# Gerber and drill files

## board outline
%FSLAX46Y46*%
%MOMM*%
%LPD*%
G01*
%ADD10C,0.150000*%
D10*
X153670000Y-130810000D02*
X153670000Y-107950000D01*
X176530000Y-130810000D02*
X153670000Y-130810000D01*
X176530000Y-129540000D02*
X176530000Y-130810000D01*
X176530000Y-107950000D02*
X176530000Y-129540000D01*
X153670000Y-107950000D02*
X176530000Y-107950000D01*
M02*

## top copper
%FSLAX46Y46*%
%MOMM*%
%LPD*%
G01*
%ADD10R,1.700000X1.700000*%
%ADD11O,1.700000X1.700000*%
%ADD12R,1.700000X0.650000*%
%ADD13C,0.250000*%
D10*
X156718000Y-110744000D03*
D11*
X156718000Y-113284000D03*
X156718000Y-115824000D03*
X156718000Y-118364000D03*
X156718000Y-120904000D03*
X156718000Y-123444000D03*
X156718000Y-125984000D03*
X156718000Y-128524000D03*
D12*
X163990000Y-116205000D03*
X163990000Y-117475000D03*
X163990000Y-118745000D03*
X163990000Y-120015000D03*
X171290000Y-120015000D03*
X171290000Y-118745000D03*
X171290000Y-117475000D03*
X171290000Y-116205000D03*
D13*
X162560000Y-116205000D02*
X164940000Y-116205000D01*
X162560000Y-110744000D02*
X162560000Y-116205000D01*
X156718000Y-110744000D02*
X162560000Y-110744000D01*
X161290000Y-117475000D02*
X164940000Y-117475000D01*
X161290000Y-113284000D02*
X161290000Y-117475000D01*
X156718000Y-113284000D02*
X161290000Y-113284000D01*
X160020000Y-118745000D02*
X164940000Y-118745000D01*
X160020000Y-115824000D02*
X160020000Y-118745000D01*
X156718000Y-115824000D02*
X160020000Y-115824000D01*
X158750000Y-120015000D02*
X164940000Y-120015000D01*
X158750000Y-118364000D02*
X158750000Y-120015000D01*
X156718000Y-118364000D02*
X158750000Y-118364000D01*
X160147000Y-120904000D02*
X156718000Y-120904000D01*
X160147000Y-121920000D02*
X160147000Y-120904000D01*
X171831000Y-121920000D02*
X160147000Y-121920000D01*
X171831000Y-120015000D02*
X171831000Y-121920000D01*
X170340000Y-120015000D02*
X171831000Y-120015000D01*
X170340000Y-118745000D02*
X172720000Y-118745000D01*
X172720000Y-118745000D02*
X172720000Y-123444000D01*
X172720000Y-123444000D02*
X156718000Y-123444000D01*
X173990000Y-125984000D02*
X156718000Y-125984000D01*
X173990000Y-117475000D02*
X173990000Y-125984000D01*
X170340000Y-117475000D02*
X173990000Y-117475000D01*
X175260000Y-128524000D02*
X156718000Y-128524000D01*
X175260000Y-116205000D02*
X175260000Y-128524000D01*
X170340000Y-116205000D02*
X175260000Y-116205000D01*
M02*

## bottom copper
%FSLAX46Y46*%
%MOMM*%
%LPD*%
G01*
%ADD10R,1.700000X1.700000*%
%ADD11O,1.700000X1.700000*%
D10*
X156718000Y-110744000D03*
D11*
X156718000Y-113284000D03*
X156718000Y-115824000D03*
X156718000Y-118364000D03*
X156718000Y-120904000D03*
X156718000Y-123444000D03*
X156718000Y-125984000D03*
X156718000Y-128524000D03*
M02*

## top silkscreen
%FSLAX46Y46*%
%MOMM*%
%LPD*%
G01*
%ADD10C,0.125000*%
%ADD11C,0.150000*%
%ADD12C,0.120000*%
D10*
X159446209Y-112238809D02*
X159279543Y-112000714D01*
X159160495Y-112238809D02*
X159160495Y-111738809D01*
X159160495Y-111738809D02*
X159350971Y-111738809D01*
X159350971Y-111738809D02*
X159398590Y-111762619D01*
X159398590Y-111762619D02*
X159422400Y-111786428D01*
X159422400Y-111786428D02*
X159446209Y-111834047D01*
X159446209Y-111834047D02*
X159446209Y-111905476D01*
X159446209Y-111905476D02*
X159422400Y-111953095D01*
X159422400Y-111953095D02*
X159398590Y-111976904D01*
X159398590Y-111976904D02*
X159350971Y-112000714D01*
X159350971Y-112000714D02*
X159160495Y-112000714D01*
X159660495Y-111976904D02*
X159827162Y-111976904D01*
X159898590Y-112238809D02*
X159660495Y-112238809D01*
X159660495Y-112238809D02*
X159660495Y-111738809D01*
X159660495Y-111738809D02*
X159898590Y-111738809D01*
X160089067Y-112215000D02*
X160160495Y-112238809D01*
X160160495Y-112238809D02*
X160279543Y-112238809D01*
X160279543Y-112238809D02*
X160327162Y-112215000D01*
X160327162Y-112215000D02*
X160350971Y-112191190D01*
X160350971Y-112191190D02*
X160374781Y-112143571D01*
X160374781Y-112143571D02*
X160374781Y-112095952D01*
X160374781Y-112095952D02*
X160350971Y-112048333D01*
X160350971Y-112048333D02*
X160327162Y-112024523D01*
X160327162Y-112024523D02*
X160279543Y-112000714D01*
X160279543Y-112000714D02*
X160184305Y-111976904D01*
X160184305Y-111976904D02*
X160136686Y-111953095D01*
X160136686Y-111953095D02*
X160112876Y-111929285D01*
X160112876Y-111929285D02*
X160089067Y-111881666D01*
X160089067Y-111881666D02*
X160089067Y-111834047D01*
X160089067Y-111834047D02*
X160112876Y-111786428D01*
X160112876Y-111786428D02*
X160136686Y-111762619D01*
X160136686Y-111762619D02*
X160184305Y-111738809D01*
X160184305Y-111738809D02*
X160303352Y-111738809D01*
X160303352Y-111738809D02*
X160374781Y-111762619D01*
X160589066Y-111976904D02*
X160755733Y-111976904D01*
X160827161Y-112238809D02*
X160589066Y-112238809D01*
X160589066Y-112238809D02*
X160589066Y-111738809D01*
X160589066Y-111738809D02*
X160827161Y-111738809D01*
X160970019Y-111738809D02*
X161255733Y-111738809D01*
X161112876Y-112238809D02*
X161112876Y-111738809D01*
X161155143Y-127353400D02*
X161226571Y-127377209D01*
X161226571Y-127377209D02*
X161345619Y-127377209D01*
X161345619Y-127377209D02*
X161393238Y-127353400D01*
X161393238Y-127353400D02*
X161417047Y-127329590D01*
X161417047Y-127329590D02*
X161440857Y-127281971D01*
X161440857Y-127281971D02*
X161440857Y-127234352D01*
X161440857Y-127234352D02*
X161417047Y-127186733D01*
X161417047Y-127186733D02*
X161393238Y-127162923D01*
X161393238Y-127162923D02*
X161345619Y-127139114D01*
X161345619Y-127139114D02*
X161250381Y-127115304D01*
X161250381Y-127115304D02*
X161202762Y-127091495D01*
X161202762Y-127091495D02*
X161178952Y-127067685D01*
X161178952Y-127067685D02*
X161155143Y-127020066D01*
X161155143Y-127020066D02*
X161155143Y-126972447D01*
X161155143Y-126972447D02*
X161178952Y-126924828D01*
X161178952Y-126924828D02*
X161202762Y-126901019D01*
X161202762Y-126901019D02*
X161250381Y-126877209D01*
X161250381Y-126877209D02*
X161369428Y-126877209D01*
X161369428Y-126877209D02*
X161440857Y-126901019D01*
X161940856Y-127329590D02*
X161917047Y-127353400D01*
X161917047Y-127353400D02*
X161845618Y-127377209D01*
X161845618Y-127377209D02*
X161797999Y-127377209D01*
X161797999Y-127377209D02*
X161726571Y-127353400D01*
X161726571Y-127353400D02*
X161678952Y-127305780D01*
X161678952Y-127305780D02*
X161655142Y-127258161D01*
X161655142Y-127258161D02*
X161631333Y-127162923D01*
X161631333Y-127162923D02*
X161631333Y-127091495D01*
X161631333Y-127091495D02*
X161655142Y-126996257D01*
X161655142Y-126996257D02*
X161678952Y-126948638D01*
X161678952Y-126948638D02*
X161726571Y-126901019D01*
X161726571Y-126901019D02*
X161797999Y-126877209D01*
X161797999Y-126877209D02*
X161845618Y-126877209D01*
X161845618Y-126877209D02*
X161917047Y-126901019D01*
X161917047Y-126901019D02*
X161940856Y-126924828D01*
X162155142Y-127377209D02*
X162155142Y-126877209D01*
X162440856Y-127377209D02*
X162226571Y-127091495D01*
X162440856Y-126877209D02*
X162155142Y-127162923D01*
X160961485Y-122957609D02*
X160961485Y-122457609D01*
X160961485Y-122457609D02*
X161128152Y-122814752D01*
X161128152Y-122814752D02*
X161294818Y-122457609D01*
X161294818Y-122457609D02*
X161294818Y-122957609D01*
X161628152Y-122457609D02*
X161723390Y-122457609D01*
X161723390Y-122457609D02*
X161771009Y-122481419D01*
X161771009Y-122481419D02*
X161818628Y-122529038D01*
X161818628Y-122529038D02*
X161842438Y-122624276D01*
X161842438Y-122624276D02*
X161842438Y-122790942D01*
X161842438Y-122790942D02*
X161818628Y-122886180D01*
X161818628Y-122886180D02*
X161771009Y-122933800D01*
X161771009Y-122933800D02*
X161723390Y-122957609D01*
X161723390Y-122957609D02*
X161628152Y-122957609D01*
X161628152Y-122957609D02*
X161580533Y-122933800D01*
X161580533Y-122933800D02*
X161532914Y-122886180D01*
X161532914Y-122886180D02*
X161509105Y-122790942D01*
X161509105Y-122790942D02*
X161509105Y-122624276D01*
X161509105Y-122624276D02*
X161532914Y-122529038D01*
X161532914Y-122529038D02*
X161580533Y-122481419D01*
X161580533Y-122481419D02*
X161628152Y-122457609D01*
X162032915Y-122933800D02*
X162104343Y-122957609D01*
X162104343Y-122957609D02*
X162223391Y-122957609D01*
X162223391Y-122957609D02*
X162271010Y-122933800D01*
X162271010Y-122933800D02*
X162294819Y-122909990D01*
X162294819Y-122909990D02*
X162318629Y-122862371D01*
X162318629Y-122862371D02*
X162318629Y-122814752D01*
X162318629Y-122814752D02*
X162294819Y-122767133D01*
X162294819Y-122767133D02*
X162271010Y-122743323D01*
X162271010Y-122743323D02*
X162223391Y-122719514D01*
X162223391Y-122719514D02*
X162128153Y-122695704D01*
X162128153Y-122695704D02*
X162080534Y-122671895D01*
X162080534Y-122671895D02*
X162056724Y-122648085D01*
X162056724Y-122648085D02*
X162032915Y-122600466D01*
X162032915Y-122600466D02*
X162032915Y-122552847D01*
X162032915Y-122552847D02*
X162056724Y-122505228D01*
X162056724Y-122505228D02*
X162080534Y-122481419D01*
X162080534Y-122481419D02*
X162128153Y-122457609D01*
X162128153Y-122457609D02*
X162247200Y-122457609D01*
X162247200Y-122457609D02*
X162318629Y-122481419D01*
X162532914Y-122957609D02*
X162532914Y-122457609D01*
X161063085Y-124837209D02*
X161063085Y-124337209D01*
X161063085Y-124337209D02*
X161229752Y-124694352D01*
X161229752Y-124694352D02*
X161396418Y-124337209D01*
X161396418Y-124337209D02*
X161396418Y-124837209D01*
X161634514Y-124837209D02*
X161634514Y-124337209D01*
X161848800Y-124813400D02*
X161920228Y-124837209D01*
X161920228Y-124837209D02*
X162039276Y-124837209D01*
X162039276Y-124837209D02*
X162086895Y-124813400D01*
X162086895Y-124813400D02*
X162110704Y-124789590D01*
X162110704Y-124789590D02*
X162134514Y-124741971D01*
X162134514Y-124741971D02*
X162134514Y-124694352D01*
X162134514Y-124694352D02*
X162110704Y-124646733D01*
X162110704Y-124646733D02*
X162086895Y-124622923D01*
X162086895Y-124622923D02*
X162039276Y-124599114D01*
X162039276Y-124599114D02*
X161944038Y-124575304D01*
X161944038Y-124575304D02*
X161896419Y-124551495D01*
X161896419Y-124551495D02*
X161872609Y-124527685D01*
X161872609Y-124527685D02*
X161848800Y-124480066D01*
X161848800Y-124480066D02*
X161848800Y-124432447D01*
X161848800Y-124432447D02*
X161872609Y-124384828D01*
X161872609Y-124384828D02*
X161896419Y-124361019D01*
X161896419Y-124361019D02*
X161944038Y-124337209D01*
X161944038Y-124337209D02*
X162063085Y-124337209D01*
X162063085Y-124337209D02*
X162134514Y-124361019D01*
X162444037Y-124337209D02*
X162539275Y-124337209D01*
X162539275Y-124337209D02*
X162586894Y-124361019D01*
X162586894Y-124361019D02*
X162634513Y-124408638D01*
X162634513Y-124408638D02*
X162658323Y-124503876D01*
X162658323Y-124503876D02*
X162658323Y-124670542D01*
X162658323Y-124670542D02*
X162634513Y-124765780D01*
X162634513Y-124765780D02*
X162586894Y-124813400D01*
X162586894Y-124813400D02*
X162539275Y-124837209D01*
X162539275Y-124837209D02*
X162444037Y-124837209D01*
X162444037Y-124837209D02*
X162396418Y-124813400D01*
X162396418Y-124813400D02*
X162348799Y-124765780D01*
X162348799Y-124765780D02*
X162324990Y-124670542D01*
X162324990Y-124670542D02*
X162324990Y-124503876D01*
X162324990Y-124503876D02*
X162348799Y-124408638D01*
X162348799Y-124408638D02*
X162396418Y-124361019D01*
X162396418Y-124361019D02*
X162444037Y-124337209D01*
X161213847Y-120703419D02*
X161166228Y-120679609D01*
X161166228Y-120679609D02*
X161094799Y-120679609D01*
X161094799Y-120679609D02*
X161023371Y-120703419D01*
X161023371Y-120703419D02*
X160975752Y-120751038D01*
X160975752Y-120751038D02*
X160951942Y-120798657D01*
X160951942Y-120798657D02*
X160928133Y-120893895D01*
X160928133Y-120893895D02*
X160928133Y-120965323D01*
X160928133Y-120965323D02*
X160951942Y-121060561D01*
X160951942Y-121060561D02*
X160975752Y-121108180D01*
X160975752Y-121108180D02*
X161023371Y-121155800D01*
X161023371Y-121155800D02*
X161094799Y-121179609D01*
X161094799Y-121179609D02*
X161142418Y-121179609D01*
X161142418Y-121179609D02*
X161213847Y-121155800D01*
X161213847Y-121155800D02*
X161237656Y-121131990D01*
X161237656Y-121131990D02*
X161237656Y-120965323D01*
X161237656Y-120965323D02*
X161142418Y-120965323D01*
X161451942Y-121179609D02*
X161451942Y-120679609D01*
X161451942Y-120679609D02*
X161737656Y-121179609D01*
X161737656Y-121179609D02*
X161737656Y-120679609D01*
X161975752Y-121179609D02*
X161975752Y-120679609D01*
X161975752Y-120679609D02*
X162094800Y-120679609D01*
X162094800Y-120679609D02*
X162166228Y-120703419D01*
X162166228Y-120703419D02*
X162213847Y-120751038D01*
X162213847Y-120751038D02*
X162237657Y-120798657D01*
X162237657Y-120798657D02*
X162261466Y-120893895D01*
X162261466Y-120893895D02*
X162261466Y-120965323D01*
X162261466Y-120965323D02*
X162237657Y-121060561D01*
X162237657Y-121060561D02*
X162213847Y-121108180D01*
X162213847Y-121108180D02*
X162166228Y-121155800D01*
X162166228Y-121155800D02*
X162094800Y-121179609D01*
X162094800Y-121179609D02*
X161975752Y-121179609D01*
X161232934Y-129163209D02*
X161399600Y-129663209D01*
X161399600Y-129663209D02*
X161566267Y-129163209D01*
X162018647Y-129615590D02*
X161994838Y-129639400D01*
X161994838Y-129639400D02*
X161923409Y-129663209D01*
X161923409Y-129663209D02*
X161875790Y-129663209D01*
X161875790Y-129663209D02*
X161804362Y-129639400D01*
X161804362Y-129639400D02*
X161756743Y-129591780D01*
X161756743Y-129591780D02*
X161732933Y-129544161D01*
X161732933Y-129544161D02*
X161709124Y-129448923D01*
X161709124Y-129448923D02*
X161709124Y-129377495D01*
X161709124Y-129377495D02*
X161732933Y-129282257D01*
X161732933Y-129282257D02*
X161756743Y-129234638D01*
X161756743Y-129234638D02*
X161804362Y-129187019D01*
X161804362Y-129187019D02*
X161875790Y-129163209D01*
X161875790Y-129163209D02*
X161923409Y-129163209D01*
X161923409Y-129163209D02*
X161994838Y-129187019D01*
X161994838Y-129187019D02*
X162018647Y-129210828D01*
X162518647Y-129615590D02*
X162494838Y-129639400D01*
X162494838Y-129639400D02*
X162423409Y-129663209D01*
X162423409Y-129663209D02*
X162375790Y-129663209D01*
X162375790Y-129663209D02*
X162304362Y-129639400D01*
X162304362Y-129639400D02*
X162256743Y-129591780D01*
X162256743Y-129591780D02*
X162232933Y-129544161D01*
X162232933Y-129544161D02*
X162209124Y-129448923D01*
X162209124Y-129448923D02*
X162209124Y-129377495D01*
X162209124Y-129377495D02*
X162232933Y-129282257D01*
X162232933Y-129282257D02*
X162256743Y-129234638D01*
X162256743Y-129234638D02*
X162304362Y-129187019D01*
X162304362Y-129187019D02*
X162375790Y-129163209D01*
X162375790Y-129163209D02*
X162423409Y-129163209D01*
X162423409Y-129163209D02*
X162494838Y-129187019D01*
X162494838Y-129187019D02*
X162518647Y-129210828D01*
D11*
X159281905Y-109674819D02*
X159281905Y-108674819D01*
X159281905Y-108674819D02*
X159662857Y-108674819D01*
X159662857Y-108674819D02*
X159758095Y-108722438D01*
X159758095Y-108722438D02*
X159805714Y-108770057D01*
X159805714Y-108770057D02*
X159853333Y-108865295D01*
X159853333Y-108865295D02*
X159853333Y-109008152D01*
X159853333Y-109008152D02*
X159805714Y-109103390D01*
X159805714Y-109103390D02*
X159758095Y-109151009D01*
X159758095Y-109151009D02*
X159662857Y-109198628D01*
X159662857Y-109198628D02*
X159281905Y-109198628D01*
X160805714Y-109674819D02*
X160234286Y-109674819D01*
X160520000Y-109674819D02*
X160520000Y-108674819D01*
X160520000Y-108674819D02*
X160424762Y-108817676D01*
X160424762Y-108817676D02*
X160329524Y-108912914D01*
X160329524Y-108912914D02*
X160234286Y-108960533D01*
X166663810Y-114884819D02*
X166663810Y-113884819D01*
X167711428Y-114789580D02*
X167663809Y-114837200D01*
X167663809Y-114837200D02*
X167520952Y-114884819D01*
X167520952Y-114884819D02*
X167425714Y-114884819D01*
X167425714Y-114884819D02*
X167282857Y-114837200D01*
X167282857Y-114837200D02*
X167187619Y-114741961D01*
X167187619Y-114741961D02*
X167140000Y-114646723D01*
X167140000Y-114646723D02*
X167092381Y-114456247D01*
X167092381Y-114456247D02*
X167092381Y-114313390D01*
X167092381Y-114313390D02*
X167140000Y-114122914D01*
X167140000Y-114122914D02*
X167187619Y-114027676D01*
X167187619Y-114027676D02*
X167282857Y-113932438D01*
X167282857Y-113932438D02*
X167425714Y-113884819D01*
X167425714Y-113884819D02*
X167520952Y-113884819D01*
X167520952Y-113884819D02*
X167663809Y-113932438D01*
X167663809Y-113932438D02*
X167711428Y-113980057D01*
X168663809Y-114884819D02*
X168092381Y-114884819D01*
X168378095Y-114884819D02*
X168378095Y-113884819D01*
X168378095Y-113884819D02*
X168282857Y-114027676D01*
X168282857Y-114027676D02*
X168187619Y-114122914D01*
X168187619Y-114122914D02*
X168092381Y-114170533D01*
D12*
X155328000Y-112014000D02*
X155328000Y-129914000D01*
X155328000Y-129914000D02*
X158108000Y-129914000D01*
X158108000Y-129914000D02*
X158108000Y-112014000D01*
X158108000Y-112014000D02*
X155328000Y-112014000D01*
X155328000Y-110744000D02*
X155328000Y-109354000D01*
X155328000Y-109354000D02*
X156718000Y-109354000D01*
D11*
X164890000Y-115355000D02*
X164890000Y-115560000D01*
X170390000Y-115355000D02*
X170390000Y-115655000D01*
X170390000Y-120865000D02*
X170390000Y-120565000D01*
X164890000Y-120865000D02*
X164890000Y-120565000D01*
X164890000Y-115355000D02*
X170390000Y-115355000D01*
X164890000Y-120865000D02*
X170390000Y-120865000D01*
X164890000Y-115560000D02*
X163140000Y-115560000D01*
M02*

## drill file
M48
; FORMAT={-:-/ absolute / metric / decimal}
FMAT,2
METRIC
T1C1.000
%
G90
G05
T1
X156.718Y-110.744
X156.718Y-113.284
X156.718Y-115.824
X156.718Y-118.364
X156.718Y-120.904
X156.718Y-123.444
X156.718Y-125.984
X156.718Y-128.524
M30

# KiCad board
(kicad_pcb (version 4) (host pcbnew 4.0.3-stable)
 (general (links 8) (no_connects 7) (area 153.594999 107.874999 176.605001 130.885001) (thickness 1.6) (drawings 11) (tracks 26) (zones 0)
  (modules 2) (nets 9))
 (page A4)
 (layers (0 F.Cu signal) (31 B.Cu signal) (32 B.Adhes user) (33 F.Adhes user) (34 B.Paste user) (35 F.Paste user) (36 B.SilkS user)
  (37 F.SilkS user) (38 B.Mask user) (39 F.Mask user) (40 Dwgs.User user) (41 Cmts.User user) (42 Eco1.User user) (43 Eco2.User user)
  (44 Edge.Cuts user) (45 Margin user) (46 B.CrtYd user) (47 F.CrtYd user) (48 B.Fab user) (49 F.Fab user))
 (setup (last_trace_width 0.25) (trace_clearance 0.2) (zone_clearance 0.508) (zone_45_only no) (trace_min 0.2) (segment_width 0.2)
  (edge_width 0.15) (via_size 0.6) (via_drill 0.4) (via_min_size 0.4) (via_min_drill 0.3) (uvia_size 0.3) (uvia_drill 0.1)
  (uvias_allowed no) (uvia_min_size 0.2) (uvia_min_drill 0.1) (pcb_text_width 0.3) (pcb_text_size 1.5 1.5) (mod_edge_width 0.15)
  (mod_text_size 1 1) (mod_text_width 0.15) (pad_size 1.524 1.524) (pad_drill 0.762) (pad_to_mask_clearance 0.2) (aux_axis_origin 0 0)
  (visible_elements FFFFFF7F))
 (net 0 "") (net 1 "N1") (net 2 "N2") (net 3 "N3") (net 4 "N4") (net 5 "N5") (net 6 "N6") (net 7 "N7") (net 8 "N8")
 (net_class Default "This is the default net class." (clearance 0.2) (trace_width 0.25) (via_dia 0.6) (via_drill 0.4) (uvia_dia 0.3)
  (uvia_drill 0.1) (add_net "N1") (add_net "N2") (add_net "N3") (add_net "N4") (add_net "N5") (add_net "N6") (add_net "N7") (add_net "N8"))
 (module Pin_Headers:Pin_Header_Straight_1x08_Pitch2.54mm (layer F.Cu) (at 156.718 110.744)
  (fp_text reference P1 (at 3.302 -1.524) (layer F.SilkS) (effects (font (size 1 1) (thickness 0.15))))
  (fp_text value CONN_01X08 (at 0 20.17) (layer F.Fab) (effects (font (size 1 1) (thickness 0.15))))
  (fp_line (start -1.39 1.27) (end -1.39 19.17) (layer F.SilkS) (width 0.12))
  (fp_line (start -1.39 19.17) (end 1.39 19.17) (layer F.SilkS) (width 0.12))
  (fp_line (start 1.39 19.17) (end 1.39 1.27) (layer F.SilkS) (width 0.12))
  (fp_line (start 1.39 1.27) (end -1.39 1.27) (layer F.SilkS) (width 0.12))
  (fp_line (start -1.39 0) (end -1.39 -1.39) (layer F.SilkS) (width 0.12))
  (fp_line (start -1.39 -1.39) (end 0 -1.39) (layer F.SilkS) (width 0.12))
  (pad 1 thru_hole rect (at 0 0) (size 1.7 1.7) (drill 1) (layers *.Cu *.Mask) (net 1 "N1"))
  (pad 2 thru_hole oval (at 0 2.54) (size 1.7 1.7) (drill 1) (layers *.Cu *.Mask) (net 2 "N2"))
  (pad 3 thru_hole oval (at 0 5.08) (size 1.7 1.7) (drill 1) (layers *.Cu *.Mask) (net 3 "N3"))
  (pad 4 thru_hole oval (at 0 7.62) (size 1.7 1.7) (drill 1) (layers *.Cu *.Mask) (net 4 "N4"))
  (pad 5 thru_hole oval (at 0 10.16) (size 1.7 1.7) (drill 1) (layers *.Cu *.Mask) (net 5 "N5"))
  (pad 6 thru_hole oval (at 0 12.7) (size 1.7 1.7) (drill 1) (layers *.Cu *.Mask) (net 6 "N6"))
  (pad 7 thru_hole oval (at 0 15.24) (size 1.7 1.7) (drill 1) (layers *.Cu *.Mask) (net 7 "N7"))
  (pad 8 thru_hole oval (at 0 17.78) (size 1.7 1.7) (drill 1) (layers *.Cu *.Mask) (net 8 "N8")))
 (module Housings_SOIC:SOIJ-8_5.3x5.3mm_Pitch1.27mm (layer F.Cu) (at 167.64 118.11)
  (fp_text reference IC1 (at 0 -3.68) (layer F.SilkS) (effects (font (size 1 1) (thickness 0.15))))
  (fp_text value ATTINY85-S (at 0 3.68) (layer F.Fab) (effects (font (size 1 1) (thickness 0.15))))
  (fp_line (start -2.75 -2.755) (end -2.75 -2.55) (layer F.SilkS) (width 0.15))
  (fp_line (start 2.75 -2.755) (end 2.75 -2.455) (layer F.SilkS) (width 0.15))
  (fp_line (start 2.75 2.755) (end 2.75 2.455) (layer F.SilkS) (width 0.15))
  (fp_line (start -2.75 2.755) (end -2.75 2.455) (layer F.SilkS) (width 0.15))
  (fp_line (start -2.75 -2.755) (end 2.75 -2.755) (layer F.SilkS) (width 0.15))
  (fp_line (start -2.75 2.755) (end 2.75 2.755) (layer F.SilkS) (width 0.15))
  (fp_line (start -2.75 -2.55) (end -4.5 -2.55) (layer F.SilkS) (width 0.15))
  (pad 1 smd rect (at -3.65 -1.905) (size 1.7 0.65) (layers F.Cu F.Paste F.Mask) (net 1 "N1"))
  (pad 2 smd rect (at -3.65 -0.635) (size 1.7 0.65) (layers F.Cu F.Paste F.Mask) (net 2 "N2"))
  (pad 3 smd rect (at -3.65 0.635) (size 1.7 0.65) (layers F.Cu F.Paste F.Mask) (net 3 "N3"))
  (pad 4 smd rect (at -3.65 1.905) (size 1.7 0.65) (layers F.Cu F.Paste F.Mask) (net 4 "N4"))
  (pad 5 smd rect (at 3.65 1.905) (size 1.7 0.65) (layers F.Cu F.Paste F.Mask) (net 5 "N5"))
  (pad 6 smd rect (at 3.65 0.635) (size 1.7 0.65) (layers F.Cu F.Paste F.Mask) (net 6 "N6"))
  (pad 7 smd rect (at 3.65 -0.635) (size 1.7 0.65) (layers F.Cu F.Paste F.Mask) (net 7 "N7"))
  (pad 8 smd rect (at 3.65 -1.905) (size 1.7 0.65) (layers F.Cu F.Paste F.Mask) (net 8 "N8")))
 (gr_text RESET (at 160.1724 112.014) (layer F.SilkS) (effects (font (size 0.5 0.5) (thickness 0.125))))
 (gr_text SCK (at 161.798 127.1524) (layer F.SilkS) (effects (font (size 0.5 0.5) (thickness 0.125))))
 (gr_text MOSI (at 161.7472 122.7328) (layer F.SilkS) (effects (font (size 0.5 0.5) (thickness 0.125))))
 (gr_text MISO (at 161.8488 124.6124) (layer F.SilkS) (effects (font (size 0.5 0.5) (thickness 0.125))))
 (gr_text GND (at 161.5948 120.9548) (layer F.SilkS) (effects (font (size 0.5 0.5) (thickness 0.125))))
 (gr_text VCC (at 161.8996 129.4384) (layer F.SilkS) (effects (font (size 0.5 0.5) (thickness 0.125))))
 (gr_line (start 153.67 130.81) (end 153.67 107.95) (layer Edge.Cuts) (width 0.15))
 (gr_line (start 176.53 130.81) (end 153.67 130.81) (layer Edge.Cuts) (width 0.15))
 (gr_line (start 176.53 129.54) (end 176.53 130.81) (layer Edge.Cuts) (width 0.15))
 (gr_line (start 176.53 107.95) (end 176.53 129.54) (layer Edge.Cuts) (width 0.15))
 (gr_line (start 153.67 107.95) (end 176.53 107.95) (layer Edge.Cuts) (width 0.15))
 (segment (start 162.56 116.205) (end 164.94 116.205) (width 0.25) (layer F.Cu) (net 1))
 (segment (start 162.56 110.744) (end 162.56 116.205) (width 0.25) (layer F.Cu) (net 1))
 (segment (start 156.718 110.744) (end 162.56 110.744) (width 0.25) (layer F.Cu) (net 1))
 (segment (start 161.29 117.475) (end 164.94 117.475) (width 0.25) (layer F.Cu) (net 2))
 (segment (start 161.29 113.284) (end 161.29 117.475) (width 0.25) (layer F.Cu) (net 2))
 (segment (start 156.718 113.284) (end 161.29 113.284) (width 0.25) (layer F.Cu) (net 2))
 (segment (start 160.02 118.745) (end 164.94 118.745) (width 0.25) (layer F.Cu) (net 3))
 (segment (start 160.02 115.824) (end 160.02 118.745) (width 0.25) (layer F.Cu) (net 3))
 (segment (start 156.718 115.824) (end 160.02 115.824) (width 0.25) (layer F.Cu) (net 3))
 (segment (start 158.75 120.015) (end 164.94 120.015) (width 0.25) (layer F.Cu) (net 4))
 (segment (start 158.75 118.364) (end 158.75 120.015) (width 0.25) (layer F.Cu) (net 4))
 (segment (start 156.718 118.364) (end 158.75 118.364) (width 0.25) (layer F.Cu) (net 4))
 (segment (start 160.147 120.904) (end 156.718 120.904) (width 0.25) (layer F.Cu) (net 5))
 (segment (start 160.147 121.92) (end 160.147 120.904) (width 0.25) (layer F.Cu) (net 5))
 (segment (start 171.831 121.92) (end 160.147 121.92) (width 0.25) (layer F.Cu) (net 5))
 (segment (start 171.831 120.015) (end 171.831 121.92) (width 0.25) (layer F.Cu) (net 5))
 (segment (start 170.34 120.015) (end 171.831 120.015) (width 0.25) (layer F.Cu) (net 5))
 (segment (start 170.34 118.745) (end 172.72 118.745) (width 0.25) (layer F.Cu) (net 6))
 (segment (start 172.72 118.745) (end 172.72 123.444) (width 0.25) (layer F.Cu) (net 6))
 (segment (start 172.72 123.444) (end 156.718 123.444) (width 0.25) (layer F.Cu) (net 6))
 (segment (start 173.99 125.984) (end 156.718 125.984) (width 0.25) (layer F.Cu) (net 7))
 (segment (start 173.99 117.475) (end 173.99 125.984) (width 0.25) (layer F.Cu) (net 7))
 (segment (start 170.34 117.475) (end 173.99 117.475) (width 0.25) (layer F.Cu) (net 7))
 (segment (start 175.26 128.524) (end 156.718 128.524) (width 0.25) (layer F.Cu) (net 8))
 (segment (start 175.26 116.205) (end 175.26 128.524) (width 0.25) (layer F.Cu) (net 8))
 (segment (start 170.34 116.205) (end 175.26 116.205) (width 0.25) (layer F.Cu) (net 8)))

